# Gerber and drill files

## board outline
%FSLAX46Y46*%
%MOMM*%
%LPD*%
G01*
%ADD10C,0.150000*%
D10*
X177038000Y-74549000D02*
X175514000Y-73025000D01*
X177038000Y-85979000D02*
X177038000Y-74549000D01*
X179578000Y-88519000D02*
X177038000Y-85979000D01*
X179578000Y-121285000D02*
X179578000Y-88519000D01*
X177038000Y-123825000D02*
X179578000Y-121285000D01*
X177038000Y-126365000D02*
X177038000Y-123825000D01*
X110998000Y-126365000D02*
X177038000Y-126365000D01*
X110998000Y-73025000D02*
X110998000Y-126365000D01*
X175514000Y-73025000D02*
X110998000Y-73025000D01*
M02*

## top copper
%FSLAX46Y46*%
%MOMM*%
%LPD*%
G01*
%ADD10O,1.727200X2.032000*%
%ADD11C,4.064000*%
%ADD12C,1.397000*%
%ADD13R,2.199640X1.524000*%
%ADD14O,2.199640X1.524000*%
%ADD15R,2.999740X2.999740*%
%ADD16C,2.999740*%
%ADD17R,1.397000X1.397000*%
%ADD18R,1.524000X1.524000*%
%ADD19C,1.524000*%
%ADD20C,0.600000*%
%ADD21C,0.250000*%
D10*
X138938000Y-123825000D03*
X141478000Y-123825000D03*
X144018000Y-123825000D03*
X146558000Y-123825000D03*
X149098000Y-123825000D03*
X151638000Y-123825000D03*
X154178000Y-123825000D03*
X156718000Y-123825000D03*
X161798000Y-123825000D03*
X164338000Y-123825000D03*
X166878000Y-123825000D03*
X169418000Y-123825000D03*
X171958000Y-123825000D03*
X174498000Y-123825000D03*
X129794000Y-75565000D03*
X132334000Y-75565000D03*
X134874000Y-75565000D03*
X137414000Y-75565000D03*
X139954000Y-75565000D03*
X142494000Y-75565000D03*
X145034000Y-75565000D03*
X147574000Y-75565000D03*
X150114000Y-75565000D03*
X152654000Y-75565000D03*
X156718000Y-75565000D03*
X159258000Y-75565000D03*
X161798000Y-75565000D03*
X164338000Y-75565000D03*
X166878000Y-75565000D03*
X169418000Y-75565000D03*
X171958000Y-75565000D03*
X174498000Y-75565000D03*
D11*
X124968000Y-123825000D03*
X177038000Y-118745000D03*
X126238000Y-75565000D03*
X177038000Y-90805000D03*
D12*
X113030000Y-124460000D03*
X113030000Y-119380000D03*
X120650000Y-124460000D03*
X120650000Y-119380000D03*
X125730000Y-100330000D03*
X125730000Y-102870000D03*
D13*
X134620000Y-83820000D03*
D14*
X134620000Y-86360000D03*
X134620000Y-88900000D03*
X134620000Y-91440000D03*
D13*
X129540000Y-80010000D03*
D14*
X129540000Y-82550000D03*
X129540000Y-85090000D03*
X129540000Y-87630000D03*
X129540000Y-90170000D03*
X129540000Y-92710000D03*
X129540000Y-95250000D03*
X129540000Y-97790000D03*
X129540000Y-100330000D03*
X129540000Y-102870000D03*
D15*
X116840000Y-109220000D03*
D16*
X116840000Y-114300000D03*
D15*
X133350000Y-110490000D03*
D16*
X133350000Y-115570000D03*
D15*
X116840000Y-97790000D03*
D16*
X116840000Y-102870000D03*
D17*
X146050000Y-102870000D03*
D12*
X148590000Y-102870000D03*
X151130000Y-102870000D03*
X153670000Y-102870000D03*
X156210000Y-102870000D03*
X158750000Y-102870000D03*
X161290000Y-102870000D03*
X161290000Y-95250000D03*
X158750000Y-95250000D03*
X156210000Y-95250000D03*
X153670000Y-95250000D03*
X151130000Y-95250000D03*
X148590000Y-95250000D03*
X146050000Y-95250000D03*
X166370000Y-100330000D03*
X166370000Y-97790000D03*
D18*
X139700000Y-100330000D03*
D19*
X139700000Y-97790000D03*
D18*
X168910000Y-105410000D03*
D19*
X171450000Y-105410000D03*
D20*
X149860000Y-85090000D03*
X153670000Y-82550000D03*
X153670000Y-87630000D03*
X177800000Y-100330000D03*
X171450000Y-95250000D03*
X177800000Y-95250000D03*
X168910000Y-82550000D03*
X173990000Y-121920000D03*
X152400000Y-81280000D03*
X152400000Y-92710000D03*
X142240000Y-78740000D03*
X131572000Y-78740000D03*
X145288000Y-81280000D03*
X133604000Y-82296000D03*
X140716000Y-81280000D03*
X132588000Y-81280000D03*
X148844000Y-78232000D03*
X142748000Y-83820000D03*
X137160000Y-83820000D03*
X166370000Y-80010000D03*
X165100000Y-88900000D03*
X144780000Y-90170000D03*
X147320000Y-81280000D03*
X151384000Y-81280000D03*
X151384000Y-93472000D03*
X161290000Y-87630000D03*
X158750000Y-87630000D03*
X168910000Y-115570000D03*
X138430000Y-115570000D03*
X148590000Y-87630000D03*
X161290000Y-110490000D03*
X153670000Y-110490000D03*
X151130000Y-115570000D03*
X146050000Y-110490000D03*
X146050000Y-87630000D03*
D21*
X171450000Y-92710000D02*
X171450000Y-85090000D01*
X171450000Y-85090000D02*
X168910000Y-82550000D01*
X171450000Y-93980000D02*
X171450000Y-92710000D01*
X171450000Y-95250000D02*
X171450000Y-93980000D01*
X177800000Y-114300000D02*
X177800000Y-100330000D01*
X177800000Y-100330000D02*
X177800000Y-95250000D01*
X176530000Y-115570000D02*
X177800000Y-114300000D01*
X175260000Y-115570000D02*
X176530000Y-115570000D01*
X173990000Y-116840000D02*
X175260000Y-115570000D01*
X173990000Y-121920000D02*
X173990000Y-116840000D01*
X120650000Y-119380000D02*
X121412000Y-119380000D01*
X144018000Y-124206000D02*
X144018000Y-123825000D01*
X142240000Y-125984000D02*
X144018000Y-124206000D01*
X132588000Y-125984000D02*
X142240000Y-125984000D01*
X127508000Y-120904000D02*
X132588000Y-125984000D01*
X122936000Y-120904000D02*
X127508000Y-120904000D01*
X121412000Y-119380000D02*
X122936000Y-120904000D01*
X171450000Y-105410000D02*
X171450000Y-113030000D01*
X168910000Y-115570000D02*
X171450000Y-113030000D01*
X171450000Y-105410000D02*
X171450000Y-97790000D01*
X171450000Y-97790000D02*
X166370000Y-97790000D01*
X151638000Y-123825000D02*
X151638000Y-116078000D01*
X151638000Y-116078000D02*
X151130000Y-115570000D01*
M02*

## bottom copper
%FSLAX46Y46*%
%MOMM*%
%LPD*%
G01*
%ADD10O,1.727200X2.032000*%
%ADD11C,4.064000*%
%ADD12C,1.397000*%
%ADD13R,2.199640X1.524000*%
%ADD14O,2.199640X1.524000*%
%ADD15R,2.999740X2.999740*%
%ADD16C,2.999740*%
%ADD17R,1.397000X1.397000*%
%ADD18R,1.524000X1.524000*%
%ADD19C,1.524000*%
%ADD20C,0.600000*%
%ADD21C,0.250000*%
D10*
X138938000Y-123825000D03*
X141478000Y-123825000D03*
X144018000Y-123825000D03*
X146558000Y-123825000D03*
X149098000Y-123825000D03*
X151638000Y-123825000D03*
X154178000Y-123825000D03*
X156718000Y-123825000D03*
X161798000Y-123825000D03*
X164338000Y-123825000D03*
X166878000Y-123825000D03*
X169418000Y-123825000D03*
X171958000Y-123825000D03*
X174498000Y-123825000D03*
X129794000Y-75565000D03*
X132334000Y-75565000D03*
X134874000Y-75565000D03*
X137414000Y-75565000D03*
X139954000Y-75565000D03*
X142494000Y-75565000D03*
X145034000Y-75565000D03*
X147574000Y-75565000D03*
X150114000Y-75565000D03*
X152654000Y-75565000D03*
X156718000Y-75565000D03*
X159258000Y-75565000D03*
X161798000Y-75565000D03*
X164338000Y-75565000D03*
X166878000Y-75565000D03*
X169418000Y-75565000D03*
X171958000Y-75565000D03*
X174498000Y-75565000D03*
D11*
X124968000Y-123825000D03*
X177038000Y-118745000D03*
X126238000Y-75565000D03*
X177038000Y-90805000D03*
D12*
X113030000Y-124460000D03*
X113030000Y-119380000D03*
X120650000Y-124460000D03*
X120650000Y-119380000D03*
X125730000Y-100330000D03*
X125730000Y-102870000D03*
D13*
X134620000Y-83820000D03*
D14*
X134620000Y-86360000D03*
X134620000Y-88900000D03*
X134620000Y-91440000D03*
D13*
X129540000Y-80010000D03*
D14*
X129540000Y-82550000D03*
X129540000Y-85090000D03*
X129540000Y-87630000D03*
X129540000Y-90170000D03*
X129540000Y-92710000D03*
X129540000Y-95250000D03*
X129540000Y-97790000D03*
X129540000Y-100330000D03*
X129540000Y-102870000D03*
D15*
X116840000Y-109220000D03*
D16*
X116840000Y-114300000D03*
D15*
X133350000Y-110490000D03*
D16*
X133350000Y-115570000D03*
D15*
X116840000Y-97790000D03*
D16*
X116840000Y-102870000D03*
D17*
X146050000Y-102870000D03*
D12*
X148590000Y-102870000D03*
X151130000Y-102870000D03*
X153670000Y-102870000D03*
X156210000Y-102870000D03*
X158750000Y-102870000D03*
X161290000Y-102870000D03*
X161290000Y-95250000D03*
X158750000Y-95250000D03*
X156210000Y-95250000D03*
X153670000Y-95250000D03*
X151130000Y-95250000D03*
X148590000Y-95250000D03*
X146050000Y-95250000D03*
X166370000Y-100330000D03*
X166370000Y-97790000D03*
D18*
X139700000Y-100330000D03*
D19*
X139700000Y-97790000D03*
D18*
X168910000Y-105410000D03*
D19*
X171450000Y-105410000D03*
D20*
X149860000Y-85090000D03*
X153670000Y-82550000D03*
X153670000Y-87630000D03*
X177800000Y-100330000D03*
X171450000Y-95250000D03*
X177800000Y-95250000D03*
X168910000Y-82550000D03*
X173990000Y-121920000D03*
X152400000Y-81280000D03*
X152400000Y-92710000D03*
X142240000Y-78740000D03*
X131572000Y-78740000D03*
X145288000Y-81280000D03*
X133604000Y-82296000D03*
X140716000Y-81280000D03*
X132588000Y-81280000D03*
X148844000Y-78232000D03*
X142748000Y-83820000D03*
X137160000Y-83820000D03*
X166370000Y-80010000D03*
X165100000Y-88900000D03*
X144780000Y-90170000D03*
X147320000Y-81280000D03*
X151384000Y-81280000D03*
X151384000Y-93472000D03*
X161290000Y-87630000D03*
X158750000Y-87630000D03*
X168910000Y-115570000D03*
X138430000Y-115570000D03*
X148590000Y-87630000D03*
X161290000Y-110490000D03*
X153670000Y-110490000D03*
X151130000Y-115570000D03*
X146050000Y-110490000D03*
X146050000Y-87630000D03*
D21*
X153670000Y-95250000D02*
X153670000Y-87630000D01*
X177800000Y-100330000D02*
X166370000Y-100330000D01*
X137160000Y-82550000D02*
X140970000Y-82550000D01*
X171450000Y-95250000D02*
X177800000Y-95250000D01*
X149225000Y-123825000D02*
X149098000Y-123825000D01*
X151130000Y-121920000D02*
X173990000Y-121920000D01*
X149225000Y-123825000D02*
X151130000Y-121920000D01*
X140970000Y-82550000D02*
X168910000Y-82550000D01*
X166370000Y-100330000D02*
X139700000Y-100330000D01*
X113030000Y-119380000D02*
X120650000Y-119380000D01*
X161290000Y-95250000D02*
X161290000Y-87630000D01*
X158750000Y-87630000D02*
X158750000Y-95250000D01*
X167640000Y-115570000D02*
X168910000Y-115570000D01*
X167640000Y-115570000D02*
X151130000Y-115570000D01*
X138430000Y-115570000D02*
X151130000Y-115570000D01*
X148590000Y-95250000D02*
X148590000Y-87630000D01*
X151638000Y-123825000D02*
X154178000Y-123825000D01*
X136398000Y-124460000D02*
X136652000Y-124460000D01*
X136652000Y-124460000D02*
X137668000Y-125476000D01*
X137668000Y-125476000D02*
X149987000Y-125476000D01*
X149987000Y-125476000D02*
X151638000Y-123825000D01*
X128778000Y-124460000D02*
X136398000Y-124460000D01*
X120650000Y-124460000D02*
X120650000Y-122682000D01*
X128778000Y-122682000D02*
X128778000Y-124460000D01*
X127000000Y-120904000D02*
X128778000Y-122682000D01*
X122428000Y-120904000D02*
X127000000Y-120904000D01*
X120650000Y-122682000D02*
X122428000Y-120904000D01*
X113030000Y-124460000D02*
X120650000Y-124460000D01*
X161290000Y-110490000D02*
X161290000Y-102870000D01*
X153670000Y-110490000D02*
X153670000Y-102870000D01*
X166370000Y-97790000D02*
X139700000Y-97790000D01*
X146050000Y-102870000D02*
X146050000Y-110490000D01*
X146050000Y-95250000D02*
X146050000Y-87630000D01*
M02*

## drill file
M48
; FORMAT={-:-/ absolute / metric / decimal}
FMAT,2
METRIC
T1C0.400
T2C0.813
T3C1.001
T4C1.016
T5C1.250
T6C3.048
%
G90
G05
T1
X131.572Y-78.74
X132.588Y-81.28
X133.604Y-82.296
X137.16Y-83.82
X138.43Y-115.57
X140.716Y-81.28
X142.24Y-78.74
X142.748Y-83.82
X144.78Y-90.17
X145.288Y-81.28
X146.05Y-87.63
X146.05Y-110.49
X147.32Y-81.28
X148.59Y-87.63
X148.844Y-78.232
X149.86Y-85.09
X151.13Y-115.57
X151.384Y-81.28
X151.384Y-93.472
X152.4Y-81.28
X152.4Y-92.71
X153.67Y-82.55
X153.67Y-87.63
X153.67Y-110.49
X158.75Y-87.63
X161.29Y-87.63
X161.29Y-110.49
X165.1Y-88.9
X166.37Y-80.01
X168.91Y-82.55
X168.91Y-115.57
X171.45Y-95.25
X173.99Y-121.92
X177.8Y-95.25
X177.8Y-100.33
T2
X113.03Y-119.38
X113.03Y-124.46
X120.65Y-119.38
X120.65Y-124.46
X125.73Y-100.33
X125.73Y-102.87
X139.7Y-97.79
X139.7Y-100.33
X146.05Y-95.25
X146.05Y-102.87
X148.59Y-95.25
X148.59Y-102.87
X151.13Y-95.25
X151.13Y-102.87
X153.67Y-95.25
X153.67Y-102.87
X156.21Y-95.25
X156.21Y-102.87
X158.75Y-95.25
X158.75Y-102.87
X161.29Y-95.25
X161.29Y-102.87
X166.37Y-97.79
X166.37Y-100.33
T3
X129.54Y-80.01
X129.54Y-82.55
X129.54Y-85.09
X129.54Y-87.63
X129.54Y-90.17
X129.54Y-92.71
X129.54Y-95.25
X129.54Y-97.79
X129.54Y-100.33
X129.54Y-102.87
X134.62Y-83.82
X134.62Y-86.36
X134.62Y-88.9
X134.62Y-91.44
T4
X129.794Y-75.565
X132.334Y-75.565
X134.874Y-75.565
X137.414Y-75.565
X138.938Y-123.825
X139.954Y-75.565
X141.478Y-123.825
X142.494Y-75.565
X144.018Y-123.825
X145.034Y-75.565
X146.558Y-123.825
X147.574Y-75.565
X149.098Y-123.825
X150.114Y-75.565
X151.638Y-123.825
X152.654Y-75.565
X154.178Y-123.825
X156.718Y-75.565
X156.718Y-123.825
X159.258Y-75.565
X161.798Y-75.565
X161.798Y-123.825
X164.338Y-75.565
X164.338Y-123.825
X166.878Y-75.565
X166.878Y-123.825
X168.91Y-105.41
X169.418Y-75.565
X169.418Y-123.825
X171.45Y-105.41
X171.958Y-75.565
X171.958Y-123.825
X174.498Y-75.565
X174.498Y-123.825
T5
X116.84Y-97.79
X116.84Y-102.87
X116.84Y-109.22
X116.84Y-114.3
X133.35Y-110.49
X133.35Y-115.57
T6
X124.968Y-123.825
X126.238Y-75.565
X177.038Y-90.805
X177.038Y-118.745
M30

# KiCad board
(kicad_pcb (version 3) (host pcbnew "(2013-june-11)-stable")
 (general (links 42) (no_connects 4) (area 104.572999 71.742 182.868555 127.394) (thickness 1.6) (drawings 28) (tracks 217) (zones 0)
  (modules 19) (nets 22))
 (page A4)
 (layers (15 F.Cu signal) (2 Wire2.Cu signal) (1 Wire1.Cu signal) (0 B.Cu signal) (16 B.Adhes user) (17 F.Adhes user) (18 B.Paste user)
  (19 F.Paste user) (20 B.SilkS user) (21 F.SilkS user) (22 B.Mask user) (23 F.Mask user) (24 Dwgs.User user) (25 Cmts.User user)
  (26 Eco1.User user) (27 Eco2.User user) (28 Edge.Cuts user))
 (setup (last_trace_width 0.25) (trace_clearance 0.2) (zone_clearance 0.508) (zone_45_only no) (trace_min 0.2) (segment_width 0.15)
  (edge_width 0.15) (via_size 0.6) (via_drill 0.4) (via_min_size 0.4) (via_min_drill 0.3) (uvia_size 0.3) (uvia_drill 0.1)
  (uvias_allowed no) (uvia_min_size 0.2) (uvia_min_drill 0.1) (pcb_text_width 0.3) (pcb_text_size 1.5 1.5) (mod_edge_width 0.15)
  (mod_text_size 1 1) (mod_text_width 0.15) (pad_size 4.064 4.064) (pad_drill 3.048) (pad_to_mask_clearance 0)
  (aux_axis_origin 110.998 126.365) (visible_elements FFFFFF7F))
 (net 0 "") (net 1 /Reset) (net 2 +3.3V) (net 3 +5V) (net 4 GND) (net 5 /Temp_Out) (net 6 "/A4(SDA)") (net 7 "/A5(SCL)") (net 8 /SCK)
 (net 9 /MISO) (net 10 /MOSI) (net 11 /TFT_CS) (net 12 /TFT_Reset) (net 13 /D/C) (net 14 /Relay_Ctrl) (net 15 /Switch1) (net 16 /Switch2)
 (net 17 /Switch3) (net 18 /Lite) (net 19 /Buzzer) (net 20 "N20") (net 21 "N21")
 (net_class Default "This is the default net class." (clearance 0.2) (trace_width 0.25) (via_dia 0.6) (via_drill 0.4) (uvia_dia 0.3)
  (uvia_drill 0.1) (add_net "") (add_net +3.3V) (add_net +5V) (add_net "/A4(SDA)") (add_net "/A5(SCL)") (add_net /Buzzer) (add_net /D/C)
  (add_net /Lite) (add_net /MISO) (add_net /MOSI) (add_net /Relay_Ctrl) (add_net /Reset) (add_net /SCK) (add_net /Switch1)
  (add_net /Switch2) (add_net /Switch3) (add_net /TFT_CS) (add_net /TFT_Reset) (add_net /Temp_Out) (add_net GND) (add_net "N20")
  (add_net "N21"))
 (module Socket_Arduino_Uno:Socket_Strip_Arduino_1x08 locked (layer F.Cu) (at 138.938 123.825)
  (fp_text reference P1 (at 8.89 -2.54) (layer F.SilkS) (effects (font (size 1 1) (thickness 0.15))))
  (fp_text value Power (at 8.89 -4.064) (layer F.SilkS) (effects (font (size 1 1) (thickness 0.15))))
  (pad 1 thru_hole oval (at 0 0) (size 1.7272 2.032) (drill 1.016) (layers *.Cu *.Mask F.SilkS))
  (pad 2 thru_hole oval (at 2.54 0) (size 1.7272 2.032) (drill 1.016) (layers *.Cu *.Mask F.SilkS))
  (pad 3 thru_hole oval (at 5.08 0) (size 1.7272 2.032) (drill 1.016) (layers *.Cu *.Mask F.SilkS) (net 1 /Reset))
  (pad 4 thru_hole oval (at 7.62 0) (size 1.7272 2.032) (drill 1.016) (layers *.Cu *.Mask F.SilkS) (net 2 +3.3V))
  (pad 5 thru_hole oval (at 10.16 0) (size 1.7272 2.032) (drill 1.016) (layers *.Cu *.Mask F.SilkS) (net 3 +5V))
  (pad 6 thru_hole oval (at 12.7 0) (size 1.7272 2.032) (drill 1.016) (layers *.Cu *.Mask F.SilkS) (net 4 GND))
  (pad 7 thru_hole oval (at 15.24 0) (size 1.7272 2.032) (drill 1.016) (layers *.Cu *.Mask F.SilkS) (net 4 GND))
  (pad 8 thru_hole oval (at 17.78 0) (size 1.7272 2.032) (drill 1.016) (layers *.Cu *.Mask F.SilkS)))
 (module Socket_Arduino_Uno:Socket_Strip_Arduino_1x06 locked (layer F.Cu) (at 161.798 123.825)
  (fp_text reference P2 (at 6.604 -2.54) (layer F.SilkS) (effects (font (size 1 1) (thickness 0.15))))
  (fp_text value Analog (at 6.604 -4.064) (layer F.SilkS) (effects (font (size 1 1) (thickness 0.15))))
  (pad 1 thru_hole oval (at 0 0) (size 1.7272 2.032) (drill 1.016) (layers *.Cu *.Mask F.SilkS) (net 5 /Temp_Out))
  (pad 2 thru_hole oval (at 2.54 0) (size 1.7272 2.032) (drill 1.016) (layers *.Cu *.Mask F.SilkS))
  (pad 3 thru_hole oval (at 5.08 0) (size 1.7272 2.032) (drill 1.016) (layers *.Cu *.Mask F.SilkS))
  (pad 4 thru_hole oval (at 7.62 0) (size 1.7272 2.032) (drill 1.016) (layers *.Cu *.Mask F.SilkS))
  (pad 5 thru_hole oval (at 10.16 0) (size 1.7272 2.032) (drill 1.016) (layers *.Cu *.Mask F.SilkS) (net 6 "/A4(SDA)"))
  (pad 6 thru_hole oval (at 12.7 0) (size 1.7272 2.032) (drill 1.016) (layers *.Cu *.Mask F.SilkS) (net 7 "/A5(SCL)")))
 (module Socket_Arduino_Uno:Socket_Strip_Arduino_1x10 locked (layer F.Cu) (at 129.794 75.565)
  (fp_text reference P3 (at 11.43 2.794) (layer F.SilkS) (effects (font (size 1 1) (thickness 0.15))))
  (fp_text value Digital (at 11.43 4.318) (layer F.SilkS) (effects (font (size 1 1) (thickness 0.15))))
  (pad 1 thru_hole oval (at 0 0) (size 1.7272 2.032) (drill 1.016) (layers *.Cu *.Mask F.SilkS) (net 7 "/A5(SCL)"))
  (pad 2 thru_hole oval (at 2.54 0) (size 1.7272 2.032) (drill 1.016) (layers *.Cu *.Mask F.SilkS) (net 6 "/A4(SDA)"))
  (pad 3 thru_hole oval (at 5.08 0) (size 1.7272 2.032) (drill 1.016) (layers *.Cu *.Mask F.SilkS) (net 2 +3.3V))
  (pad 4 thru_hole oval (at 7.62 0) (size 1.7272 2.032) (drill 1.016) (layers *.Cu *.Mask F.SilkS) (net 4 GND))
  (pad 5 thru_hole oval (at 10.16 0) (size 1.7272 2.032) (drill 1.016) (layers *.Cu *.Mask F.SilkS) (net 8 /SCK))
  (pad 6 thru_hole oval (at 12.7 0) (size 1.7272 2.032) (drill 1.016) (layers *.Cu *.Mask F.SilkS) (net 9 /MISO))
  (pad 7 thru_hole oval (at 15.24 0) (size 1.7272 2.032) (drill 1.016) (layers *.Cu *.Mask F.SilkS) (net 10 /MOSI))
  (pad 8 thru_hole oval (at 17.78 0) (size 1.7272 2.032) (drill 1.016) (layers *.Cu *.Mask F.SilkS) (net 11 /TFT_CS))
  (pad 9 thru_hole oval (at 20.32 0) (size 1.7272 2.032) (drill 1.016) (layers *.Cu *.Mask F.SilkS) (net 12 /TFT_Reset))
  (pad 10 thru_hole oval (at 22.86 0) (size 1.7272 2.032) (drill 1.016) (layers *.Cu *.Mask F.SilkS) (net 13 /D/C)))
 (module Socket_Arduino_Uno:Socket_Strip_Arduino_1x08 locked (layer F.Cu) (at 156.718 75.565)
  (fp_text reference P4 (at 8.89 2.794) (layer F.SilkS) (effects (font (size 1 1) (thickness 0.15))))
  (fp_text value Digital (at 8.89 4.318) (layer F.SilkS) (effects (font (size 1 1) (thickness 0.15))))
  (pad 1 thru_hole oval (at 0 0) (size 1.7272 2.032) (drill 1.016) (layers *.Cu *.Mask F.SilkS) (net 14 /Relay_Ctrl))
  (pad 2 thru_hole oval (at 2.54 0) (size 1.7272 2.032) (drill 1.016) (layers *.Cu *.Mask F.SilkS) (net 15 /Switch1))
  (pad 3 thru_hole oval (at 5.08 0) (size 1.7272 2.032) (drill 1.016) (layers *.Cu *.Mask F.SilkS) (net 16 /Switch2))
  (pad 4 thru_hole oval (at 7.62 0) (size 1.7272 2.032) (drill 1.016) (layers *.Cu *.Mask F.SilkS) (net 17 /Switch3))
  (pad 5 thru_hole oval (at 10.16 0) (size 1.7272 2.032) (drill 1.016) (layers *.Cu *.Mask F.SilkS) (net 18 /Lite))
  (pad 6 thru_hole oval (at 12.7 0) (size 1.7272 2.032) (drill 1.016) (layers *.Cu *.Mask F.SilkS) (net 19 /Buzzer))
  (pad 7 thru_hole oval (at 15.24 0) (size 1.7272 2.032) (drill 1.016) (layers *.Cu *.Mask F.SilkS))
  (pad 8 thru_hole oval (at 17.78 0) (size 1.7272 2.032) (drill 1.016) (layers *.Cu *.Mask F.SilkS)))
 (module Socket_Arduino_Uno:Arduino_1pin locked (layer F.Cu) (at 124.968 123.825)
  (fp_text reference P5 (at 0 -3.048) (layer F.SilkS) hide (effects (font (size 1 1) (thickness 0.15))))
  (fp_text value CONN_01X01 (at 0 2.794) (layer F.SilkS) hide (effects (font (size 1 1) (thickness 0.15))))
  (pad 1 thru_hole circle (at 0 0) (size 4.064 4.064) (drill 3.048) (layers *.Cu *.Mask F.SilkS)))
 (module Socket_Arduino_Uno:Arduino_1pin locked (layer F.Cu) (at 177.038 118.745)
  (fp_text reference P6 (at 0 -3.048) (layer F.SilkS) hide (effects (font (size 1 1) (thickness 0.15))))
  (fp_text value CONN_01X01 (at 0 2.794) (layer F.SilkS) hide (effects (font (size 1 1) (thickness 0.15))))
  (pad 1 thru_hole circle (at 0 0) (size 4.064 4.064) (drill 3.048) (layers *.Cu *.Mask F.SilkS)))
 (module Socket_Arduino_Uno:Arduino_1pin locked (layer F.Cu) (at 126.238 75.565)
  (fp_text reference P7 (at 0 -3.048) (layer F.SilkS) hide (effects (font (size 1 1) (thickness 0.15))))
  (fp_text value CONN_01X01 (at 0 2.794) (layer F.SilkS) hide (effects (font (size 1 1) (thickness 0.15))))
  (pad 1 thru_hole circle (at 0 0) (size 4.064 4.064) (drill 3.048) (layers *.Cu *.Mask F.SilkS)))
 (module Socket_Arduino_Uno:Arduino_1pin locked (layer F.Cu) (at 177.038 90.805)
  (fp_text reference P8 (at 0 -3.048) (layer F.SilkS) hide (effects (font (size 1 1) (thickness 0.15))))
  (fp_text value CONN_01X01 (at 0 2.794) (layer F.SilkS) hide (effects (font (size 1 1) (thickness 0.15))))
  (pad 1 thru_hole circle (at 0 0) (size 4.064 4.064) (drill 3.048) (layers *.Cu *.Mask F.SilkS)))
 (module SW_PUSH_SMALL (layer F.Cu) (at 116.84 121.92 180)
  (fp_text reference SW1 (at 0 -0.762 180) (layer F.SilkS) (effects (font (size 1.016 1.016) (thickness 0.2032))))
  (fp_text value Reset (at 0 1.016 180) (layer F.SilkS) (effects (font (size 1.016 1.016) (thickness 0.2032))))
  (pad 1 thru_hole circle (at 3.81 -2.54 180) (size 1.397 1.397) (drill 0.8128) (layers *.Cu *.Mask F.SilkS) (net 4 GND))
  (pad 2 thru_hole circle (at 3.81 2.54 180) (size 1.397 1.397) (drill 0.8128) (layers *.Cu *.Mask F.SilkS) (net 1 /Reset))
  (pad 1 thru_hole circle (at -3.81 -2.54 180) (size 1.397 1.397) (drill 0.8128) (layers *.Cu *.Mask F.SilkS) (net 4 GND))
  (pad 2 thru_hole circle (at -3.81 2.54 180) (size 1.397 1.397) (drill 0.8128) (layers *.Cu *.Mask F.SilkS) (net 1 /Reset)))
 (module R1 (layer F.Cu) (at 125.73 101.6 270) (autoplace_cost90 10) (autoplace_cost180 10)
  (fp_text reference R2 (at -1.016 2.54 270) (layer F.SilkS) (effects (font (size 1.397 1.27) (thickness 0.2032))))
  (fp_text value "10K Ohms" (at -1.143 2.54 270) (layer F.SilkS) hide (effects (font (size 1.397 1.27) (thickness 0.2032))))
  (pad 1 thru_hole circle (at -1.27 0 270) (size 1.397 1.397) (drill 0.8128) (layers *.Cu *.Mask F.SilkS) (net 14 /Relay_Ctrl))
  (pad 2 thru_hole circle (at 1.27 0 270) (size 1.397 1.397) (drill 0.8128) (layers *.Cu *.Mask F.SilkS) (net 4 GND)))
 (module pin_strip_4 (layer F.Cu) (at 134.62 87.63 270)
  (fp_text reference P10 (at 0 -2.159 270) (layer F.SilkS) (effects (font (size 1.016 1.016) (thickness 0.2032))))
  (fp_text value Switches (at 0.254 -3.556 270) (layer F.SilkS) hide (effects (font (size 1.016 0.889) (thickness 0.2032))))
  (pad 1 thru_hole rect (at -3.81 0 270) (size 1.524 2.19964) (drill 1.00076) (layers *.Cu *.Mask F.SilkS) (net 15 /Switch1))
  (pad 2 thru_hole oval (at -1.27 0 270) (size 1.524 2.19964) (drill 1.00076) (layers *.Cu *.Mask F.SilkS) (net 16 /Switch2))
  (pad 3 thru_hole oval (at 1.27 0 270) (size 1.524 2.19964) (drill 1.00076) (layers *.Cu *.Mask F.SilkS) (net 17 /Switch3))
  (pad 4 thru_hole oval (at 3.81 0 270) (size 1.524 2.19964) (drill 1.00076) (layers *.Cu *.Mask F.SilkS) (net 4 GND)))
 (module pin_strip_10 (layer F.Cu) (at 129.54 91.44 270)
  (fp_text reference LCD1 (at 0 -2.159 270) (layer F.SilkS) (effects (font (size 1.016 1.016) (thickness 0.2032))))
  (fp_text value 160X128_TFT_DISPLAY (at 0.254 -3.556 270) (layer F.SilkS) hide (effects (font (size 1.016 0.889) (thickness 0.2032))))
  (pad 1 thru_hole rect (at -11.43 0 270) (size 1.524 2.19964) (drill 1.00076) (layers *.Cu *.Mask F.SilkS) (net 18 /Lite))
  (pad 2 thru_hole oval (at -8.89 0 270) (size 1.524 2.19964) (drill 1.00076) (layers *.Cu *.Mask F.SilkS) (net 9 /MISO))
  (pad 3 thru_hole oval (at -6.35 0 270) (size 1.524 2.19964) (drill 1.00076) (layers *.Cu *.Mask F.SilkS) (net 8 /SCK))
  (pad 4 thru_hole oval (at -3.81 0 270) (size 1.524 2.19964) (drill 1.00076) (layers *.Cu *.Mask F.SilkS) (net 10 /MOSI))
  (pad 5 thru_hole oval (at -1.27 0 270) (size 1.524 2.19964) (drill 1.00076) (layers *.Cu *.Mask F.SilkS) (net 11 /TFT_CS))
  (pad 6 thru_hole oval (at 1.27 0 270) (size 1.524 2.19964) (drill 1.00076) (layers *.Cu *.Mask F.SilkS))
  (pad 7 thru_hole oval (at 3.81 0 270) (size 1.524 2.19964) (drill 1.00076) (layers *.Cu *.Mask F.SilkS) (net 13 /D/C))
  (pad 8 thru_hole oval (at 6.35 0 270) (size 1.524 2.19964) (drill 1.00076) (layers *.Cu *.Mask F.SilkS) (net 12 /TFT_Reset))
  (pad 9 thru_hole oval (at 8.89 0 270) (size 1.524 2.19964) (drill 1.00076) (layers *.Cu *.Mask F.SilkS) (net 3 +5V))
  (pad 10 thru_hole oval (at 11.43 0 270) (size 1.524 2.19964) (drill 1.00076) (layers *.Cu *.Mask F.SilkS) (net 4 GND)))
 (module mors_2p (layer F.Cu) (at 116.84 111.76 270)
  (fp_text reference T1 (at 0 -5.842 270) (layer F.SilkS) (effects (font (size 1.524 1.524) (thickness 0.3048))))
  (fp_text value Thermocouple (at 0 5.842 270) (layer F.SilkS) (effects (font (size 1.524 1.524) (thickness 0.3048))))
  (pad 1 thru_hole rect (at -2.54 0 270) (size 2.99974 2.99974) (drill 1.24968) (layers *.Cu *.Mask F.SilkS) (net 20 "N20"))
  (pad 2 thru_hole circle (at 2.54 0 270) (size 2.99974 2.99974) (drill 1.24968) (layers *.Cu *.Mask F.SilkS) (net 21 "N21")))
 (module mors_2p (layer F.Cu) (at 133.35 113.03 270)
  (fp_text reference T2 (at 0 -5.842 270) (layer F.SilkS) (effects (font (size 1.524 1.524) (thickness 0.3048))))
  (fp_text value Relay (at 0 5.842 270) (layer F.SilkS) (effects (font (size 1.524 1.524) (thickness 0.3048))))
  (pad 1 thru_hole rect (at -2.54 0 270) (size 2.99974 2.99974) (drill 1.24968) (layers *.Cu *.Mask F.SilkS) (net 14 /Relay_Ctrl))
  (pad 2 thru_hole circle (at 2.54 0 270) (size 2.99974 2.99974) (drill 1.24968) (layers *.Cu *.Mask F.SilkS) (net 4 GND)))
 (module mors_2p (layer F.Cu) (at 116.84 100.33 270)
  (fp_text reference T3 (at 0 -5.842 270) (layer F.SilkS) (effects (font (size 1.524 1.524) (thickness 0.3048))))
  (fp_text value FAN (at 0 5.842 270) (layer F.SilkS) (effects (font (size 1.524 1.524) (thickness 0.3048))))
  (pad 1 thru_hole rect (at -2.54 0 270) (size 2.99974 2.99974) (drill 1.24968) (layers *.Cu *.Mask F.SilkS) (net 3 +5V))
  (pad 2 thru_hole circle (at 2.54 0 270) (size 2.99974 2.99974) (drill 1.24968) (layers *.Cu *.Mask F.SilkS) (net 4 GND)))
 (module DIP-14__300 (layer F.Cu) (at 153.67 99.06)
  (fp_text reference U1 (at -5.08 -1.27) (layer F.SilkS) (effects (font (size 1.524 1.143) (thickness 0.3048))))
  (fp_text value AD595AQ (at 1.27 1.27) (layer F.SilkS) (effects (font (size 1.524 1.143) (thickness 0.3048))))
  (pad 1 thru_hole rect (at -7.62 3.81) (size 1.397 1.397) (drill 0.8128) (layers *.Cu *.Mask F.SilkS) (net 20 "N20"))
  (pad 2 thru_hole circle (at -5.08 3.81) (size 1.397 1.397) (drill 0.8128) (layers *.Cu *.Mask F.SilkS))
  (pad 3 thru_hole circle (at -2.54 3.81) (size 1.397 1.397) (drill 0.8128) (layers *.Cu *.Mask F.SilkS))
  (pad 4 thru_hole circle (at 0 3.81) (size 1.397 1.397) (drill 0.8128) (layers *.Cu *.Mask F.SilkS) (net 4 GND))
  (pad 5 thru_hole circle (at 2.54 3.81) (size 1.397 1.397) (drill 0.8128) (layers *.Cu *.Mask F.SilkS))
  (pad 6 thru_hole circle (at 5.08 3.81) (size 1.397 1.397) (drill 0.8128) (layers *.Cu *.Mask F.SilkS))
  (pad 7 thru_hole circle (at 7.62 3.81) (size 1.397 1.397) (drill 0.8128) (layers *.Cu *.Mask F.SilkS) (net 4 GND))
  (pad 8 thru_hole circle (at 7.62 -3.81) (size 1.397 1.397) (drill 0.8128) (layers *.Cu *.Mask F.SilkS) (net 5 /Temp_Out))
  (pad 9 thru_hole circle (at 5.08 -3.81) (size 1.397 1.397) (drill 0.8128) (layers *.Cu *.Mask F.SilkS) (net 5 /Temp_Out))
  (pad 10 thru_hole circle (at 2.54 -3.81) (size 1.397 1.397) (drill 0.8128) (layers *.Cu *.Mask F.SilkS))
  (pad 11 thru_hole circle (at 0 -3.81) (size 1.397 1.397) (drill 0.8128) (layers *.Cu *.Mask F.SilkS) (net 3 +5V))
  (pad 12 thru_hole circle (at -2.54 -3.81) (size 1.397 1.397) (drill 0.8128) (layers *.Cu *.Mask F.SilkS))
  (pad 13 thru_hole circle (at -5.08 -3.81) (size 1.397 1.397) (drill 0.8128) (layers *.Cu *.Mask F.SilkS) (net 4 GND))
  (pad 14 thru_hole circle (at -7.62 -3.81) (size 1.397 1.397) (drill 0.8128) (layers *.Cu *.Mask F.SilkS) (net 21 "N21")))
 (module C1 (layer F.Cu) (at 166.37 99.06 90)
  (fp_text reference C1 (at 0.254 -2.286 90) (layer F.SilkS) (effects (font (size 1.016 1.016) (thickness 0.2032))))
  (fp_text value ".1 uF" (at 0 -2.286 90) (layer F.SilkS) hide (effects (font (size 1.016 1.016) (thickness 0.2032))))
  (pad 1 thru_hole circle (at -1.27 0 90) (size 1.397 1.397) (drill 0.8128) (layers *.Cu *.Mask F.SilkS) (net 3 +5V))
  (pad 2 thru_hole circle (at 1.27 0 90) (size 1.397 1.397) (drill 0.8128) (layers *.Cu *.Mask F.SilkS) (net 4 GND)))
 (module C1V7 (layer F.Cu) (at 139.7 99.06 90)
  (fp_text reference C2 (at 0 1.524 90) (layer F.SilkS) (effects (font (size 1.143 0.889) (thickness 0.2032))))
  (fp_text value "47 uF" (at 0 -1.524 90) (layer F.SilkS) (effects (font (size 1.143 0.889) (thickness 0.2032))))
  (pad 1 thru_hole rect (at -1.27 0 90) (size 1.524 1.524) (drill 0.8128) (layers *.Cu *.Mask F.SilkS) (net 3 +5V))
  (pad 2 thru_hole circle (at 1.27 0 90) (size 1.524 1.524) (drill 0.8128) (layers *.Cu *.Mask F.SilkS) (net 4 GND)))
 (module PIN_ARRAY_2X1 (layer F.Cu) (at 170.18 105.41)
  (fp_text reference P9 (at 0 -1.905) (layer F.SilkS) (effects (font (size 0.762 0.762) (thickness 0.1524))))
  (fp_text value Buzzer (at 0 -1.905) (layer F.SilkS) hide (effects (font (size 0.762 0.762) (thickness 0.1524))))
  (pad 1 thru_hole rect (at -1.27 0) (size 1.524 1.524) (drill 1.016) (layers *.Cu *.Mask F.SilkS) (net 19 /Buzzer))
  (pad 2 thru_hole circle (at 1.27 0) (size 1.524 1.524) (drill 1.016) (layers *.Cu *.Mask F.SilkS) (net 4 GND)))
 (gr_line (start 177.038 74.549) (end 175.514 73.025) (angle 90) (layer Edge.Cuts) (width 0.15))
 (gr_line (start 177.038 85.979) (end 177.038 74.549) (angle 90) (layer Edge.Cuts) (width 0.15))
 (gr_line (start 179.578 88.519) (end 177.038 85.979) (angle 90) (layer Edge.Cuts) (width 0.15))
 (gr_line (start 179.578 121.285) (end 179.578 88.519) (angle 90) (layer Edge.Cuts) (width 0.15))
 (gr_line (start 177.038 123.825) (end 179.578 121.285) (angle 90) (layer Edge.Cuts) (width 0.15))
 (gr_line (start 177.038 126.365) (end 177.038 123.825) (angle 90) (layer Edge.Cuts) (width 0.15))
 (gr_line (start 110.998 126.365) (end 177.038 126.365) (angle 90) (layer Edge.Cuts) (width 0.15))
 (gr_line (start 110.998 73.025) (end 110.998 126.365) (angle 90) (layer Edge.Cuts) (width 0.15))
 (gr_line (start 175.514 73.025) (end 110.998 73.025) (angle 90) (layer Edge.Cuts) (width 0.15))
 (segment (start 149.86 85.09) (end 139.7 85.09) (width 0.25) (layer Wire2.Cu) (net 2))
 (segment (start 146.558 112.522) (end 149.86 109.22) (width 0.25) (layer Wire1.Cu) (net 2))
 (segment (start 149.86 109.22) (end 149.86 85.09) (width 0.25) (layer Wire1.Cu) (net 2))
 (via (at 149.86 85.09) (size 0.6) (layers F.Cu B.Cu) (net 2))
 (segment (start 146.558 123.825) (end 146.558 112.522) (width 0.25) (layer Wire1.Cu) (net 2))
 (segment (start 134.874 77.216) (end 134.874 75.565) (width 0.25) (layer Wire2.Cu) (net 2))
 (segment (start 134.62 77.47) (end 134.874 77.216) (width 0.25) (layer Wire2.Cu) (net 2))
 (segment (start 137.16 77.47) (end 134.62 77.47) (width 0.25) (layer Wire2.Cu) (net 2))
 (segment (start 139.7 80.01) (end 137.16 77.47) (width 0.25) (layer Wire2.Cu) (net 2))
 (segment (start 139.7 85.09) (end 139.7 80.01) (width 0.25) (layer Wire2.Cu) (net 2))
 (segment (start 153.67 95.25) (end 153.67 87.63) (width 0.25) (layer B.Cu) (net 3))
 (via (at 153.67 82.55) (size 0.6) (layers F.Cu B.Cu) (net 3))
 (segment (start 153.67 87.63) (end 153.67 82.55) (width 0.25) (layer Wire1.Cu) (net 3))
 (via (at 153.67 87.63) (size 0.6) (layers F.Cu B.Cu) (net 3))
 (segment (start 177.8 100.33) (end 166.37 100.33) (width 0.25) (layer B.Cu) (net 3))
 (via (at 177.8 100.33) (size 0.6) (layers F.Cu B.Cu) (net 3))
 (segment (start 129.54 100.33) (end 128.27 100.33) (width 0.25) (layer Wire2.Cu) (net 3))
 (segment (start 125.73 97.79) (end 116.84 97.79) (width 0.25) (layer Wire2.Cu) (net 3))
 (segment (start 128.27 100.33) (end 125.73 97.79) (width 0.25) (layer Wire2.Cu) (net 3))
 (segment (start 139.7 100.33) (end 129.54 100.33) (width 0.25) (layer Wire2.Cu) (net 3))
 (segment (start 137.16 82.55) (end 140.97 82.55) (width 0.25) (layer B.Cu) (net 3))
 (via (at 171.45 95.25) (size 0.6) (layers F.Cu B.Cu) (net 3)) (via (at 177.8 95.25) (size 0.6) (layers F.Cu B.Cu) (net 3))
 (segment (start 171.45 95.25) (end 177.8 95.25) (width 0.25) (layer B.Cu) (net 3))
 (segment (start 149.225 123.825) (end 149.098 123.825) (width 0.25) (layer B.Cu) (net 3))
 (via (at 168.91 82.55) (size 0.6) (layers F.Cu B.Cu) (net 3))
 (segment (start 171.45 92.71) (end 171.45 85.09) (width 0.25) (layer F.Cu) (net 3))
 (segment (start 171.45 85.09) (end 168.91 82.55) (width 0.25) (layer F.Cu) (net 3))
 (segment (start 171.45 93.98) (end 171.45 92.71) (width 0.25) (layer F.Cu) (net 3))
 (segment (start 171.45 95.25) (end 171.45 93.98) (width 0.25) (layer F.Cu) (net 3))
 (segment (start 177.8 114.3) (end 177.8 100.33) (width 0.25) (layer F.Cu) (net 3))
 (segment (start 177.8 100.33) (end 177.8 95.25) (width 0.25) (layer F.Cu) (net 3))
 (segment (start 176.53 115.57) (end 177.8 114.3) (width 0.25) (layer F.Cu) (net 3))
 (segment (start 175.26 115.57) (end 176.53 115.57) (width 0.25) (layer F.Cu) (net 3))
 (segment (start 173.99 116.84) (end 175.26 115.57) (width 0.25) (layer F.Cu) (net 3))
 (segment (start 173.99 121.92) (end 173.99 116.84) (width 0.25) (layer F.Cu) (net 3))
 (via (at 173.99 121.92) (size 0.6) (layers F.Cu B.Cu) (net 3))
 (segment (start 151.13 121.92) (end 173.99 121.92) (width 0.25) (layer B.Cu) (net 3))
 (segment (start 149.225 123.825) (end 151.13 121.92) (width 0.25) (layer B.Cu) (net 3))
 (segment (start 140.97 82.55) (end 168.91 82.55) (width 0.25) (layer B.Cu) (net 3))
 (segment (start 166.37 100.33) (end 139.7 100.33) (width 0.25) (layer B.Cu) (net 3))
 (segment (start 168.91 105.41) (end 168.91 103.505) (width 0.25) (layer Wire1.Cu) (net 19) (status 400000))
 (segment (start 169.926 76.073) (end 169.418 75.565) (width 0.25) (layer Wire1.Cu) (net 19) (status C00000))
 (segment (start 169.926 102.489) (end 169.926 76.073) (width 0.25) (layer Wire1.Cu) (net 19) (status 800000))
 (segment (start 168.91 103.505) (end 169.926 102.489) (width 0.25) (layer Wire1.Cu) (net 19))
 (segment (start 152.398011 92.460057) (end 152.398011 92.708011) (width 0.25) (layer Wire2.Cu) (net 13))
 (segment (start 136.906 95.25) (end 140.287967 92.556403) (width 0.25) (layer Wire2.Cu) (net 13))
 (segment (start 140.287967 92.556403) (end 152.398011 92.460057) (width 0.25) (layer Wire2.Cu) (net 13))
 (segment (start 129.54 95.25) (end 136.906 95.25) (width 0.25) (layer Wire2.Cu) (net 13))
 (segment (start 152.654 81.026) (end 152.654 75.565) (width 0.25) (layer Wire2.Cu) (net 13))
 (segment (start 152.4 81.28) (end 152.654 81.026) (width 0.25) (layer Wire2.Cu) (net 13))
 (via (at 152.4 81.28) (size 0.6) (layers F.Cu B.Cu) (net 13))
 (segment (start 152.4 92.71) (end 152.4 81.28) (width 0.25) (layer Wire1.Cu) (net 13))
 (via (at 152.4 92.71) (size 0.6) (layers F.Cu B.Cu) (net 13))
 (segment (start 152.398011 92.708011) (end 152.4 92.71) (width 0.25) (layer Wire2.Cu) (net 13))
 (segment (start 129.54 80.01) (end 163.83 80.01) (width 0.25) (layer Wire1.Cu) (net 18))
 (segment (start 166.878 76.962) (end 166.878 75.565) (width 0.25) (layer Wire1.Cu) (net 18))
 (segment (start 163.83 80.01) (end 166.878 76.962) (width 0.25) (layer Wire1.Cu) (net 18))
 (segment (start 129.54 82.55) (end 130.81 82.55) (width 0.25) (layer Wire2.Cu) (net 9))
 (segment (start 142.494 78.486) (end 142.494 75.565) (width 0.25) (layer Wire2.Cu) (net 9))
 (segment (start 142.24 78.74) (end 142.494 78.486) (width 0.25) (layer Wire2.Cu) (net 9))
 (via (at 142.24 78.74) (size 0.6) (layers F.Cu B.Cu) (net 9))
 (segment (start 131.572 78.74) (end 142.24 78.74) (width 0.25) (layer Wire1.Cu) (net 9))
 (via (at 131.572 78.74) (size 0.6) (layers F.Cu B.Cu) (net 9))
 (segment (start 131.572 81.788) (end 131.572 78.74) (width 0.25) (layer Wire2.Cu) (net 9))
 (segment (start 130.81 82.55) (end 131.572 81.788) (width 0.25) (layer Wire2.Cu) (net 9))
 (segment (start 129.54 87.63) (end 130.302 87.63) (width 0.25) (layer Wire2.Cu) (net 10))
 (segment (start 145.034 81.026) (end 145.034 75.565) (width 0.25) (layer Wire2.Cu) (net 10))
 (segment (start 145.288 81.28) (end 145.034 81.026) (width 0.25) (layer Wire2.Cu) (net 10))
 (via (at 145.288 81.28) (size 0.6) (layers F.Cu B.Cu) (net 10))
 (segment (start 144.78 81.28) (end 145.288 81.28) (width 0.25) (layer Wire1.Cu) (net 10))
 (segment (start 143.764 82.296) (end 144.78 81.28) (width 0.25) (layer Wire1.Cu) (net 10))
 (segment (start 133.604 82.296) (end 143.764 82.296) (width 0.25) (layer Wire1.Cu) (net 10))
 (via (at 133.604 82.296) (size 0.6) (layers F.Cu B.Cu) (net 10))
 (segment (start 133.096 82.804) (end 133.604 82.296) (width 0.25) (layer Wire2.Cu) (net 10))
 (segment (start 133.096 84.836) (end 133.096 82.804) (width 0.25) (layer Wire2.Cu) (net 10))
 (segment (start 130.302 87.63) (end 133.096 84.836) (width 0.25) (layer Wire2.Cu) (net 10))
 (segment (start 133.35 110.49) (end 127 110.49) (width 0.25) (layer Wire1.Cu) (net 14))
 (segment (start 123.19 102.87) (end 125.73 100.33) (width 0.25) (layer Wire1.Cu) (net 14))
 (segment (start 123.19 106.68) (end 123.19 102.87) (width 0.25) (layer Wire1.Cu) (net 14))
 (segment (start 127 110.49) (end 123.19 106.68) (width 0.25) (layer Wire1.Cu) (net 14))
 (segment (start 125.73 100.33) (end 125.73 80.01) (width 0.25) (layer Wire1.Cu) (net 14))
 (segment (start 154.813 77.47) (end 156.718 75.565) (width 0.25) (layer Wire1.Cu) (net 14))
 (segment (start 128.27 77.47) (end 154.813 77.47) (width 0.25) (layer Wire1.Cu) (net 14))
 (segment (start 125.73 80.01) (end 128.27 77.47) (width 0.25) (layer Wire1.Cu) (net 14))
 (segment (start 120.65 119.38) (end 121.412 119.38) (width 0.25) (layer F.Cu) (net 1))
 (segment (start 144.018 124.206) (end 144.018 123.825) (width 0.25) (layer F.Cu) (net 1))
 (segment (start 142.24 125.984) (end 144.018 124.206) (width 0.25) (layer F.Cu) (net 1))
 (segment (start 132.588 125.984) (end 142.24 125.984) (width 0.25) (layer F.Cu) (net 1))
 (segment (start 127.508 120.904) (end 132.588 125.984) (width 0.25) (layer F.Cu) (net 1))
 (segment (start 122.936 120.904) (end 127.508 120.904) (width 0.25) (layer F.Cu) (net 1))
 (segment (start 121.412 119.38) (end 122.936 120.904) (width 0.25) (layer F.Cu) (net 1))
 (segment (start 113.03 119.38) (end 120.65 119.38) (width 0.25) (layer B.Cu) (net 1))
 (segment (start 129.54 85.09) (end 129.794 85.09) (width 0.25) (layer Wire2.Cu) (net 8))
 (segment (start 139.954 76.962) (end 139.954 75.565) (width 0.25) (layer Wire2.Cu) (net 8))
 (segment (start 140.716 77.724) (end 139.954 76.962) (width 0.25) (layer Wire2.Cu) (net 8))
 (segment (start 140.716 81.28) (end 140.716 77.724) (width 0.25) (layer Wire2.Cu) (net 8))
 (via (at 140.716 81.28) (size 0.6) (layers F.Cu B.Cu) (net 8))
 (segment (start 132.588 81.28) (end 140.716 81.28) (width 0.25) (layer Wire1.Cu) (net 8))
 (via (at 132.588 81.28) (size 0.6) (layers F.Cu B.Cu) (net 8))
 (segment (start 132.588 82.296) (end 132.588 81.28) (width 0.25) (layer Wire2.Cu) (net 8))
 (segment (start 129.794 85.09) (end 132.588 82.296) (width 0.25) (layer Wire2.Cu) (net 8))
 (segment (start 134.62 83.82) (end 137.16 83.82) (width 0.25) (layer Wire2.Cu) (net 15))
 (segment (start 159.258 77.978) (end 159.258 75.565) (width 0.25) (layer Wire1.Cu) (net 15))
 (segment (start 158.496 78.74) (end 159.258 77.978) (width 0.25) (layer Wire1.Cu) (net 15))
 (segment (start 149.352 78.74) (end 158.496 78.74) (width 0.25) (layer Wire1.Cu) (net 15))
 (segment (start 148.844 78.232) (end 149.352 78.74) (width 0.25) (layer Wire1.Cu) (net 15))
 (via (at 148.844 78.232) (size 0.6) (layers F.Cu B.Cu) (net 15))
 (segment (start 148.844 82.804) (end 148.844 78.232) (width 0.25) (layer Wire2.Cu) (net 15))
 (segment (start 149.86 83.82) (end 148.844 82.804) (width 0.25) (layer Wire2.Cu) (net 15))
 (segment (start 142.748 83.82) (end 149.86 83.82) (width 0.25) (layer Wire2.Cu) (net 15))
 (via (at 142.748 83.82) (size 0.6) (layers F.Cu B.Cu) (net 15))
 (segment (start 137.16 83.82) (end 142.748 83.82) (width 0.25) (layer Wire1.Cu) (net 15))
 (via (at 137.16 83.82) (size 0.6) (layers F.Cu B.Cu) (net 15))
 (segment (start 134.62 86.36) (end 160.02 86.36) (width 0.25) (layer Wire2.Cu) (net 16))
 (segment (start 161.798 84.582) (end 161.798 75.565) (width 0.25) (layer Wire2.Cu) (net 16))
 (segment (start 160.02 86.36) (end 161.798 84.582) (width 0.25) (layer Wire2.Cu) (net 16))
 (segment (start 134.62 88.9) (end 165.1 88.9) (width 0.25) (layer Wire2.Cu) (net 17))
 (segment (start 164.338 77.978) (end 164.338 75.565) (width 0.25) (layer Wire2.Cu) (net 17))
 (segment (start 166.37 80.01) (end 164.338 77.978) (width 0.25) (layer Wire2.Cu) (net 17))
 (via (at 166.37 80.01) (size 0.6) (layers F.Cu B.Cu) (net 17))
 (segment (start 166.37 87.63) (end 166.37 80.01) (width 0.25) (layer Wire1.Cu) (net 17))
 (segment (start 165.1 88.9) (end 166.37 87.63) (width 0.25) (layer Wire1.Cu) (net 17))
 (via (at 165.1 88.9) (size 0.6) (layers F.Cu B.Cu) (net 17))
 (segment (start 144.78 86.36) (end 144.78 85.09) (width 0.25) (layer Wire1.Cu) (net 11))
 (segment (start 137.16 90.17) (end 144.78 90.17) (width 0.25) (layer Wire2.Cu) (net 11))
 (via (at 144.78 90.17) (size 0.6) (layers F.Cu B.Cu) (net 11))
 (segment (start 144.78 90.17) (end 144.78 86.36) (width 0.25) (layer Wire1.Cu) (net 11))
 (segment (start 144.78 85.09) (end 146.05 83.82) (width 0.25) (layer Wire1.Cu) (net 11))
 (segment (start 146.05 83.608333) (end 146.05 83.82) (width 0.25) (layer Wire1.Cu) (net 11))
 (segment (start 146.05 83.82) (end 146.05 83.608333) (width 0.25) (layer Wire1.Cu) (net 11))
 (segment (start 146.05 83.608333) (end 147.32 81.28) (width 0.25) (layer Wire1.Cu) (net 11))
 (segment (start 147.574 81.026) (end 147.574 75.565) (width 0.25) (layer Wire2.Cu) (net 11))
 (segment (start 147.32 81.28) (end 147.574 81.026) (width 0.25) (layer Wire2.Cu) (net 11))
 (via (at 147.32 81.28) (size 0.6) (layers F.Cu B.Cu) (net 11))
 (segment (start 129.54 90.17) (end 137.16 90.17) (width 0.25) (layer Wire2.Cu) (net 11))
 (segment (start 137.16 90.17) (end 137.414 90.17) (width 0.25) (layer Wire2.Cu) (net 11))
 (segment (start 129.54 97.79) (end 135.89 97.79) (width 0.25) (layer Wire2.Cu) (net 12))
 (segment (start 150.114 80.01) (end 150.114 75.565) (width 0.25) (layer Wire2.Cu) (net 12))
 (segment (start 151.384 81.28) (end 150.114 80.01) (width 0.25) (layer Wire2.Cu) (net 12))
 (via (at 151.384 81.28) (size 0.6) (layers F.Cu B.Cu) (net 12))
 (segment (start 151.384 93.472) (end 151.384 81.28) (width 0.25) (layer Wire1.Cu) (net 12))
 (via (at 151.384 93.472) (size 0.6) (layers F.Cu B.Cu) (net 12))
 (segment (start 140.716 93.472) (end 151.384 93.472) (width 0.25) (layer Wire2.Cu) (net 12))
 (segment (start 135.89 97.79) (end 140.716 93.472) (width 0.25) (layer Wire2.Cu) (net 12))
 (segment (start 161.29 87.63) (end 162.56 87.63) (width 0.25) (layer Wire1.Cu) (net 5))
 (segment (start 161.798 122.682) (end 161.798 123.825) (width 0.25) (layer Wire1.Cu) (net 5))
 (segment (start 163.83 120.65) (end 161.798 122.682) (width 0.25) (layer Wire1.Cu) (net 5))
 (segment (start 163.83 88.9) (end 163.83 120.65) (width 0.25) (layer Wire1.Cu) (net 5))
 (segment (start 162.56 87.63) (end 163.83 88.9) (width 0.25) (layer Wire1.Cu) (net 5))
 (segment (start 158.75 87.63) (end 161.29 87.63) (width 0.25) (layer Wire2.Cu) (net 5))
 (segment (start 161.29 95.25) (end 161.29 87.63) (width 0.25) (layer B.Cu) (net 5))
 (via (at 161.29 87.63) (size 0.6) (layers F.Cu B.Cu) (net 5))
 (segment (start 158.75 87.63) (end 158.75 95.25) (width 0.25) (layer B.Cu) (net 5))
 (via (at 158.75 87.63) (size 0.6) (layers F.Cu B.Cu) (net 5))
 (segment (start 171.45 105.41) (end 171.45 113.03) (width 0.25) (layer F.Cu) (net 4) (status 400000))
 (segment (start 167.64 115.57) (end 168.91 115.57) (width 0.25) (layer B.Cu) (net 4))
 (segment (start 168.91 115.57) (end 171.45 113.03) (width 0.25) (layer F.Cu) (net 4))
 (via (at 168.91 115.57) (size 0.6) (layers F.Cu B.Cu) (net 4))
 (segment (start 167.64 115.57) (end 151.13 115.57) (width 0.25) (layer B.Cu) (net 4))
 (segment (start 171.45 105.41) (end 171.45 97.79) (width 0.25) (layer F.Cu) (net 4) (status 400000))
 (segment (start 171.45 97.79) (end 166.37 97.79) (width 0.25) (layer F.Cu) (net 4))
 (segment (start 133.35 115.57) (end 138.43 115.57) (width 0.25) (layer Wire2.Cu) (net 4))
 (via (at 138.43 115.57) (size 0.6) (layers F.Cu B.Cu) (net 4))
 (segment (start 138.43 115.57) (end 151.13 115.57) (width 0.25) (layer B.Cu) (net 4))
 (segment (start 133.35 115.57) (end 137.16 111.76) (width 0.25) (layer Wire1.Cu) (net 4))
 (segment (start 137.16 107.95) (end 132.08 102.87) (width 0.25) (layer Wire1.Cu) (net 4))
 (segment (start 137.16 111.76) (end 137.16 107.95) (width 0.25) (layer Wire1.Cu) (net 4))
 (segment (start 148.59 87.63) (end 148.59 91.44) (width 0.25) (layer Wire1.Cu) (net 4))
 (segment (start 148.59 95.25) (end 148.59 87.63) (width 0.25) (layer B.Cu) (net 4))
 (via (at 148.59 87.63) (size 0.6) (layers F.Cu B.Cu) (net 4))
 (segment (start 148.59 91.44) (end 137.16 91.44) (width 0.25) (layer Wire1.Cu) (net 4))
 (segment (start 137.414 91.44) (end 137.16 91.44) (width 0.25) (layer Wire1.Cu) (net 4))
 (segment (start 137.16 91.44) (end 134.62 91.44) (width 0.25) (layer Wire1.Cu) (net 4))
 (segment (start 151.638 123.825) (end 154.178 123.825) (width 0.25) (layer B.Cu) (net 4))
 (segment (start 134.62 91.44) (end 134.62 100.076) (width 0.25) (layer Wire1.Cu) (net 4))
 (segment (start 131.826 102.87) (end 129.54 102.87) (width 0.25) (layer Wire1.Cu) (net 4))
 (segment (start 134.62 100.076) (end 131.826 102.87) (width 0.25) (layer Wire1.Cu) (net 4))
 (segment (start 136.398 124.46) (end 136.652 124.46) (width 0.25) (layer B.Cu) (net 4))
 (segment (start 136.652 124.46) (end 137.668 125.476) (width 0.25) (layer B.Cu) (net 4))
 (segment (start 137.668 125.476) (end 149.987 125.476) (width 0.25) (layer B.Cu) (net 4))
 (segment (start 149.987 125.476) (end 151.638 123.825) (width 0.25) (layer B.Cu) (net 4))
 (segment (start 128.778 124.46) (end 136.398 124.46) (width 0.25) (layer B.Cu) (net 4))
 (segment (start 120.65 124.46) (end 120.65 122.682) (width 0.25) (layer B.Cu) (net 4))
 (segment (start 128.778 122.682) (end 128.778 124.46) (width 0.25) (layer B.Cu) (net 4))
 (segment (start 127 120.904) (end 128.778 122.682) (width 0.25) (layer B.Cu) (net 4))
 (segment (start 122.428 120.904) (end 127 120.904) (width 0.25) (layer B.Cu) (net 4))
 (segment (start 120.65 122.682) (end 122.428 120.904) (width 0.25) (layer B.Cu) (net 4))
 (segment (start 113.03 124.46) (end 120.65 124.46) (width 0.25) (layer B.Cu) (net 4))
 (segment (start 125.73 102.87) (end 116.84 102.87) (width 0.25) (layer Wire2.Cu) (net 4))
 (segment (start 129.54 102.87) (end 125.73 102.87) (width 0.25) (layer Wire2.Cu) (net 4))
 (segment (start 139.7 97.79) (end 139.7 96.52) (width 0.25) (layer Wire1.Cu) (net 4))
 (segment (start 139.7 96.52) (end 134.62 91.44) (width 0.25) (layer Wire1.Cu) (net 4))
 (segment (start 153.67 110.49) (end 161.29 110.49) (width 0.25) (layer Wire2.Cu) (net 4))
 (via (at 161.29 110.49) (size 0.6) (layers F.Cu B.Cu) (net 4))
 (segment (start 161.29 110.49) (end 161.29 102.87) (width 0.25) (layer B.Cu) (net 4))
 (segment (start 153.67 113.03) (end 153.67 110.49) (width 0.25) (layer Wire1.Cu) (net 4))
 (segment (start 151.13 115.57) (end 153.67 113.03) (width 0.25) (layer Wire1.Cu) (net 4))
 (via (at 153.67 110.49) (size 0.6) (layers F.Cu B.Cu) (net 4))
 (segment (start 153.67 110.49) (end 153.67 102.87) (width 0.25) (layer B.Cu) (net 4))
 (segment (start 151.638 123.825) (end 151.638 116.078) (width 0.25) (layer F.Cu) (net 4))
 (segment (start 151.638 116.078) (end 151.13 115.57) (width 0.25) (layer F.Cu) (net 4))
 (via (at 151.13 115.57) (size 0.6) (layers F.Cu B.Cu) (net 4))
 (segment (start 166.37 97.79) (end 139.7 97.79) (width 0.25) (layer B.Cu) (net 4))
 (segment (start 146.05 102.87) (end 146.05 110.49) (width 0.25) (layer B.Cu) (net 20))
 (segment (start 119.38 111.76) (end 116.84 109.22) (width 0.25) (layer Wire2.Cu) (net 20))
 (segment (start 120.65 113.03) (end 119.38 111.76) (width 0.25) (layer Wire2.Cu) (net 20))
 (segment (start 143.51 113.03) (end 120.65 113.03) (width 0.25) (layer Wire2.Cu) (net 20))
 (segment (start 146.05 110.49) (end 143.51 113.03) (width 0.25) (layer Wire2.Cu) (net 20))
 (via (at 146.05 110.49) (size 0.6) (layers F.Cu B.Cu) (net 20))
 (segment (start 146.05 87.63) (end 133.35 87.63) (width 0.25) (layer Wire2.Cu) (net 21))
 (via (at 146.05 87.63) (size 0.6) (layers F.Cu B.Cu) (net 21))
 (segment (start 146.05 95.25) (end 146.05 87.63) (width 0.25) (layer B.Cu) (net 21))
 (segment (start 111.76 114.3) (end 116.84 114.3) (width 0.25) (layer Wire2.Cu) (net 21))
 (segment (start 111.76 88.9) (end 111.76 114.3) (width 0.25) (layer Wire2.Cu) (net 21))
 (segment (start 132.08 88.9) (end 111.76 88.9) (width 0.25) (layer Wire2.Cu) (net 21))
 (segment (start 133.35 87.63) (end 132.08 88.9) (width 0.25) (layer Wire2.Cu) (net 21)))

